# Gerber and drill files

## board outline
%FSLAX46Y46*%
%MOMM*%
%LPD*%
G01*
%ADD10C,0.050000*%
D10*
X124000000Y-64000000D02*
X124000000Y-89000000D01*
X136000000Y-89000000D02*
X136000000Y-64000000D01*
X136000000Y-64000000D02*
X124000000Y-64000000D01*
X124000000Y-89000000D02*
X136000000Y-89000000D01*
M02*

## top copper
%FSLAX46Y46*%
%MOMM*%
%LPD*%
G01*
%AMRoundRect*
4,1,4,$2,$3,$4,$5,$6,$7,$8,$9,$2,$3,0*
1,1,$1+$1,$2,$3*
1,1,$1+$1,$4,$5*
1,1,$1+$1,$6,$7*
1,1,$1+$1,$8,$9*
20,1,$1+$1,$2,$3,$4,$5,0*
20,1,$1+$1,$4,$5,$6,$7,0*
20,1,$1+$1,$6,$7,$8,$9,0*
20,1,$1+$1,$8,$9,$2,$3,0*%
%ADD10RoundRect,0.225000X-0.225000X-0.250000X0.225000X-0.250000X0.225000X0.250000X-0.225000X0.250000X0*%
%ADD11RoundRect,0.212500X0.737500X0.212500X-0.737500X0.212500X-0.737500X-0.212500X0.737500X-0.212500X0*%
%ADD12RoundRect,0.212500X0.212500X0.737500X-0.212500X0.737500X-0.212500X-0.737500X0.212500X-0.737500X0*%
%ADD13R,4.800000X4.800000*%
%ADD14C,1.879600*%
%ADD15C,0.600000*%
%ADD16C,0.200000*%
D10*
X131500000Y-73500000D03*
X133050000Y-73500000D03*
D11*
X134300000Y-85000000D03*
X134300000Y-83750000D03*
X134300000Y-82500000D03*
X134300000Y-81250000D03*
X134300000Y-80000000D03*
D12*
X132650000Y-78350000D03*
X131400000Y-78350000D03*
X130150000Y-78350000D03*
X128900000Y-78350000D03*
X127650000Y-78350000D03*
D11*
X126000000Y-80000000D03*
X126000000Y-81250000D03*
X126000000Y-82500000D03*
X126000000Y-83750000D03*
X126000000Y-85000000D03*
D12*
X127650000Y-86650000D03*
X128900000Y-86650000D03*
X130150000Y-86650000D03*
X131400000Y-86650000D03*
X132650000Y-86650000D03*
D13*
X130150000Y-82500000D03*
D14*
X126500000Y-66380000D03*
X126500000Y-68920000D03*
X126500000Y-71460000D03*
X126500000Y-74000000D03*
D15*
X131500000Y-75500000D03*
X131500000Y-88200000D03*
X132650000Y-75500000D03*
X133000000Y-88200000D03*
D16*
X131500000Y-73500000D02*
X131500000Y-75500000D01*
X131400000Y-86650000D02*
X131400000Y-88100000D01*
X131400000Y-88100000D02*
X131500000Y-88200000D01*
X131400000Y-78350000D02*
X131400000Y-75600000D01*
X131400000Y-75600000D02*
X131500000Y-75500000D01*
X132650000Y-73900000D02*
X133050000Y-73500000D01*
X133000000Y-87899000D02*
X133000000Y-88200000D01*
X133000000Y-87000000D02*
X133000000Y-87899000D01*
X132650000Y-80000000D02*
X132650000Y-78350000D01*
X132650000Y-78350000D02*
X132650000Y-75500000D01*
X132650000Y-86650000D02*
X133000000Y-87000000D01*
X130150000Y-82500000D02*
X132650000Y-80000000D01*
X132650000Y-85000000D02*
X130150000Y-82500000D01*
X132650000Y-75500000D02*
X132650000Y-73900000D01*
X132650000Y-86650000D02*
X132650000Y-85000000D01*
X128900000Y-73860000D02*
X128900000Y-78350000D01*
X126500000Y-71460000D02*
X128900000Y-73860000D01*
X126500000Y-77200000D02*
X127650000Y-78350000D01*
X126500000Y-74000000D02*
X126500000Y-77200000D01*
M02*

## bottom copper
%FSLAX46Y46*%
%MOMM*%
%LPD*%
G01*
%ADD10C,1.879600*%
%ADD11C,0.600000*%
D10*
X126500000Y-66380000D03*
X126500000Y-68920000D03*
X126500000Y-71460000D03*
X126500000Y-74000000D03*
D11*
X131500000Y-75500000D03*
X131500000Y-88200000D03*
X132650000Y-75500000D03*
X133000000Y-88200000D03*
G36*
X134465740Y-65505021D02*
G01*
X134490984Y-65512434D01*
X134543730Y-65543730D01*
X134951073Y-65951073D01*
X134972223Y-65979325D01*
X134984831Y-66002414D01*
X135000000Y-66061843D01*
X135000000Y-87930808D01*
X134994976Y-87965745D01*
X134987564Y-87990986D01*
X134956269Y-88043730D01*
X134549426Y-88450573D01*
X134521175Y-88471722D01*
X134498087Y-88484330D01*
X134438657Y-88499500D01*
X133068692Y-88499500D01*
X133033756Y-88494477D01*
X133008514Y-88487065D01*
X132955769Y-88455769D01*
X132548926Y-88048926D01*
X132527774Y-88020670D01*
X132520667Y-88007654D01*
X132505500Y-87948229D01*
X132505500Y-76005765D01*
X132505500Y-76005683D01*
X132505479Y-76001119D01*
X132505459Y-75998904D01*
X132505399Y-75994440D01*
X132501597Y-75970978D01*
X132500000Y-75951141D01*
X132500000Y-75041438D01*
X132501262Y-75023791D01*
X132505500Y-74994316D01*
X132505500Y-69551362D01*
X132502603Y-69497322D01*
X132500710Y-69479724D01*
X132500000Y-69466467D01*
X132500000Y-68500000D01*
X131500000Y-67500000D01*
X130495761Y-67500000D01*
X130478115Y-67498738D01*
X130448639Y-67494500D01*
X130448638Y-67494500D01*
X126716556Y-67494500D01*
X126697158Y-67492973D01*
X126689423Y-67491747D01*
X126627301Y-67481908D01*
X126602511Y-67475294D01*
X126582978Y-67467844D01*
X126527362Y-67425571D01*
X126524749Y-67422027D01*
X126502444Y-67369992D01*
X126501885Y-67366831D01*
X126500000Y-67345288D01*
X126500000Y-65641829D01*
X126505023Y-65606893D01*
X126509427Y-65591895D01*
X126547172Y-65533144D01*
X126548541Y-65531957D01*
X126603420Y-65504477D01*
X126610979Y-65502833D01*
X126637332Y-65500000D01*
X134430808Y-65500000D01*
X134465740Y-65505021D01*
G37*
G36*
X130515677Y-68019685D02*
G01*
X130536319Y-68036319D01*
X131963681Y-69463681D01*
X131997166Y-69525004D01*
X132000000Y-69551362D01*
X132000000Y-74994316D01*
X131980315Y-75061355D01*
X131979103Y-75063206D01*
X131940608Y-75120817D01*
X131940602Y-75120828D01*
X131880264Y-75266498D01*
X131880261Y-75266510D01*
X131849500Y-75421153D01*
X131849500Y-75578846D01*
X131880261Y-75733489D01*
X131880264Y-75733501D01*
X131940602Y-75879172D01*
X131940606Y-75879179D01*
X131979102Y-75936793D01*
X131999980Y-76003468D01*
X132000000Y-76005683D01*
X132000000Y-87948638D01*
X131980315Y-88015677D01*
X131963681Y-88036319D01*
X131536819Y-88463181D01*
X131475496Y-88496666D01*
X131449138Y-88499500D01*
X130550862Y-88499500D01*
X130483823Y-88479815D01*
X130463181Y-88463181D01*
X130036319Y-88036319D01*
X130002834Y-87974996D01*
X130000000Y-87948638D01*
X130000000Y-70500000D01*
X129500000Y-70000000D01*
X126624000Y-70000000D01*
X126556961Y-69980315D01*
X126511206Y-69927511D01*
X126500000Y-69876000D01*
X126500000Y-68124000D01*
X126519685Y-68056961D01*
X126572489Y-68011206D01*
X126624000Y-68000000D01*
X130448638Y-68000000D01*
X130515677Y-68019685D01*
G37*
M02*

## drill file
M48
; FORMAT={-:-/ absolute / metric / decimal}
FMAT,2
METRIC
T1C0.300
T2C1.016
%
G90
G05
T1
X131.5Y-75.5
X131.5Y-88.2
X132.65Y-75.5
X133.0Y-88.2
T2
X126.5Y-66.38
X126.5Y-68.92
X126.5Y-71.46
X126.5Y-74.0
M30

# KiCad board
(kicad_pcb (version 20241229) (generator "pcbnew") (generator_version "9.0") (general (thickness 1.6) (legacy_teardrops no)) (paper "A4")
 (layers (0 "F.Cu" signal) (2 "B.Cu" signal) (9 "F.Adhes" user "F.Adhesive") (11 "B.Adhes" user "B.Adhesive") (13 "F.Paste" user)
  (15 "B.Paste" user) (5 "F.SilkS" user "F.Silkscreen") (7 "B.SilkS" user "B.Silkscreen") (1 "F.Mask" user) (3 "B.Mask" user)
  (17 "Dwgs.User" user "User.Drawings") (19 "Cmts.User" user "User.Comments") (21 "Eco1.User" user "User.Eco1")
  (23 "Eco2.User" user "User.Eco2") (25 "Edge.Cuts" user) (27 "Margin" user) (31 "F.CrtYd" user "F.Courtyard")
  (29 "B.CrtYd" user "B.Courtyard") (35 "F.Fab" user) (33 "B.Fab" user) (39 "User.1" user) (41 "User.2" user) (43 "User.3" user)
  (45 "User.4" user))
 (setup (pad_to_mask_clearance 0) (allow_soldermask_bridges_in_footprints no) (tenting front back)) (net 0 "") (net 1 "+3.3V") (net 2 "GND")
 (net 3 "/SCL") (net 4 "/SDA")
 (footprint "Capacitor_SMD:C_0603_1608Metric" (layer "F.Cu") (at 132.275 73.5)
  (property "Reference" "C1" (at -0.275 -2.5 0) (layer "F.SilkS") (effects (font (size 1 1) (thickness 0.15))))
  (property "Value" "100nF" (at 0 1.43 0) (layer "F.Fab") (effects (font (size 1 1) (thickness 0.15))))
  (pad "1" smd roundrect (at -0.775 0) (size 0.9 0.95) (layers "F.Cu" "F.Mask" "F.Paste") (roundrect_rratio 0.25) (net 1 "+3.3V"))
  (pad "2" smd roundrect (at 0.775 0) (size 0.9 0.95) (layers "F.Cu" "F.Mask" "F.Paste") (roundrect_rratio 0.25) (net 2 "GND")))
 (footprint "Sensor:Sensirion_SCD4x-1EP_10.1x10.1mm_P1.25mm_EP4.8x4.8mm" (layer "F.Cu") (at 130.15 82.5 180)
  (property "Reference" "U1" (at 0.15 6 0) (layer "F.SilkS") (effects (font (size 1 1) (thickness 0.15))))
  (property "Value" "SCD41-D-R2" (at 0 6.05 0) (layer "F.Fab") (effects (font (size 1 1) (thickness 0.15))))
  (pad "" smd roundrect (at -1.2 -1.2 180) (size 1.93 1.93) (layers "F.Paste") (roundrect_rratio 0.129534))
  (pad "" smd roundrect (at -1.2 1.2 180) (size 1.93 1.93) (layers "F.Paste") (roundrect_rratio 0.129534))
  (pad "" smd roundrect (at 1.2 -1.2 180) (size 1.93 1.93) (layers "F.Paste") (roundrect_rratio 0.129534))
  (pad "" smd roundrect (at 1.2 1.2 180) (size 1.93 1.93) (layers "F.Paste") (roundrect_rratio 0.129534))
  (pad "1" smd roundrect (at -4.15 -2.5 180) (size 1.9 0.85) (layers "F.Cu" "F.Mask" "F.Paste") (roundrect_rratio 0.25))
  (pad "2" smd roundrect (at -4.15 -1.25 180) (size 1.9 0.85) (layers "F.Cu" "F.Mask" "F.Paste") (roundrect_rratio 0.25))
  (pad "3" smd roundrect (at -4.15 0 180) (size 1.9 0.85) (layers "F.Cu" "F.Mask" "F.Paste") (roundrect_rratio 0.25))
  (pad "4" smd roundrect (at -4.15 1.25 180) (size 1.9 0.85) (layers "F.Cu" "F.Mask" "F.Paste") (roundrect_rratio 0.25))
  (pad "5" smd roundrect (at -4.15 2.5 180) (size 1.9 0.85) (layers "F.Cu" "F.Mask" "F.Paste") (roundrect_rratio 0.25))
  (pad "6" smd roundrect (at -2.5 4.15 180) (size 0.85 1.9) (layers "F.Cu" "F.Mask" "F.Paste") (roundrect_rratio 0.25) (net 2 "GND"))
  (pad "7" smd roundrect (at -1.25 4.15 180) (size 0.85 1.9) (layers "F.Cu" "F.Mask" "F.Paste") (roundrect_rratio 0.25) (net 1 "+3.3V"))
  (pad "8" smd roundrect (at 0 4.15 180) (size 0.85 1.9) (layers "F.Cu" "F.Mask" "F.Paste") (roundrect_rratio 0.25))
  (pad "9" smd roundrect (at 1.25 4.15 180) (size 0.85 1.9) (layers "F.Cu" "F.Mask" "F.Paste") (roundrect_rratio 0.25) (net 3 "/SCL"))
  (pad "10" smd roundrect (at 2.5 4.15 180) (size 0.85 1.9) (layers "F.Cu" "F.Mask" "F.Paste") (roundrect_rratio 0.25) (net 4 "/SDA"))
  (pad "11" smd roundrect (at 4.15 2.5 180) (size 1.9 0.85) (layers "F.Cu" "F.Mask" "F.Paste") (roundrect_rratio 0.25))
  (pad "12" smd roundrect (at 4.15 1.25 180) (size 1.9 0.85) (layers "F.Cu" "F.Mask" "F.Paste") (roundrect_rratio 0.25))
  (pad "13" smd roundrect (at 4.15 0 180) (size 1.9 0.85) (layers "F.Cu" "F.Mask" "F.Paste") (roundrect_rratio 0.25))
  (pad "14" smd roundrect (at 4.15 -1.25 180) (size 1.9 0.85) (layers "F.Cu" "F.Mask" "F.Paste") (roundrect_rratio 0.25))
  (pad "15" smd roundrect (at 4.15 -2.5 180) (size 1.9 0.85) (layers "F.Cu" "F.Mask" "F.Paste") (roundrect_rratio 0.25))
  (pad "16" smd roundrect (at 2.5 -4.15 180) (size 0.85 1.9) (layers "F.Cu" "F.Mask" "F.Paste") (roundrect_rratio 0.25))
  (pad "17" smd roundrect (at 1.25 -4.15 180) (size 0.85 1.9) (layers "F.Cu" "F.Mask" "F.Paste") (roundrect_rratio 0.25))
  (pad "18" smd roundrect (at 0 -4.15 180) (size 0.85 1.9) (layers "F.Cu" "F.Mask" "F.Paste") (roundrect_rratio 0.25))
  (pad "19" smd roundrect (at -1.25 -4.15 180) (size 0.85 1.9) (layers "F.Cu" "F.Mask" "F.Paste") (roundrect_rratio 0.25) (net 1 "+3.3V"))
  (pad "20" smd roundrect (at -2.5 -4.15 180) (size 0.85 1.9) (layers "F.Cu" "F.Mask" "F.Paste") (roundrect_rratio 0.25) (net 2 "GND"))
  (pad "21" smd rect (at 0 0 180) (size 4.8 4.8) (layers "F.Cu" "F.Mask") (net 2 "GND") (zone_connect 2)))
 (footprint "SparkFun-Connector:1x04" (layer "F.Cu") (at 126.5 66.38 -90)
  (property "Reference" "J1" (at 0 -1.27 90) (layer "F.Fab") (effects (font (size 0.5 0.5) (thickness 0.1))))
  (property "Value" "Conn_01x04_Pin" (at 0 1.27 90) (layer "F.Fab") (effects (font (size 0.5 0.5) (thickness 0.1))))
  (pad "1" thru_hole circle (at 0 0) (size 1.8796 1.8796) (drill 1.016) (layers "*.Cu" "*.Mask") (remove_unused_layers yes)
   (keep_end_layers yes) (zone_layer_connections) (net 2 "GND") (thermal_bridge_angle 0))
  (pad "2" thru_hole circle (at 2.54 0) (size 1.8796 1.8796) (drill 1.016) (layers "*.Cu" "*.Mask") (remove_unused_layers yes)
   (keep_end_layers yes) (zone_layer_connections) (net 1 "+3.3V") (thermal_bridge_angle 0))
  (pad "3" thru_hole circle (at 5.08 0) (size 1.8796 1.8796) (drill 1.016) (layers "*.Cu" "*.Mask") (remove_unused_layers yes)
   (keep_end_layers yes) (zone_layer_connections) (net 3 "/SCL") (thermal_bridge_angle 0))
  (pad "4" thru_hole circle (at 7.62 0) (size 1.8796 1.8796) (drill 1.016) (layers "*.Cu" "*.Mask") (remove_unused_layers yes)
   (keep_end_layers yes) (zone_layer_connections) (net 4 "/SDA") (thermal_bridge_angle 0)))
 (gr_line (start 124 64) (end 124 89) (stroke (width 0.05) (type default)) (layer "Edge.Cuts"))
 (gr_line (start 136 89) (end 136 64) (stroke (width 0.05) (type default)) (layer "Edge.Cuts"))
 (gr_line (start 136 64) (end 124 64) (stroke (width 0.05) (type default)) (layer "Edge.Cuts"))
 (gr_line (start 124 89) (end 136 89) (stroke (width 0.05) (type default)) (layer "Edge.Cuts"))
 (segment (start 131.5 73.5) (end 131.5 75.5) (width 0.2) (layer "F.Cu") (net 1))
 (segment (start 131.4 86.65) (end 131.4 88.1) (width 0.2) (layer "F.Cu") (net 1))
 (segment (start 131.4 88.1) (end 131.5 88.2) (width 0.2) (layer "F.Cu") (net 1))
 (segment (start 131.4 78.35) (end 131.4 75.6) (width 0.2) (layer "F.Cu") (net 1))
 (segment (start 131.4 75.6) (end 131.5 75.5) (width 0.2) (layer "F.Cu") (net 1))
 (via (at 131.5 75.5) (size 0.6) (drill 0.3) (layers "F.Cu" "B.Cu") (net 1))
 (via (at 131.5 88.2) (size 0.6) (drill 0.3) (layers "F.Cu" "B.Cu") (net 1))
 (segment (start 132.65 73.9) (end 133.05 73.5) (width 0.2) (layer "F.Cu") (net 2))
 (segment (start 133 87.899) (end 133 88.2) (width 0.2) (layer "F.Cu") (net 2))
 (segment (start 133 87) (end 133 87.899) (width 0.2) (layer "F.Cu") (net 2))
 (segment (start 132.65 80) (end 132.65 78.35) (width 0.2) (layer "F.Cu") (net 2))
 (segment (start 132.65 78.35) (end 132.65 75.5) (width 0.2) (layer "F.Cu") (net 2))
 (segment (start 132.65 86.65) (end 133 87) (width 0.2) (layer "F.Cu") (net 2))
 (segment (start 130.15 82.5) (end 132.65 80) (width 0.2) (layer "F.Cu") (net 2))
 (segment (start 132.65 85) (end 130.15 82.5) (width 0.2) (layer "F.Cu") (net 2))
 (segment (start 132.65 75.5) (end 132.65 73.9) (width 0.2) (layer "F.Cu") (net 2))
 (segment (start 132.65 86.65) (end 132.65 85) (width 0.2) (layer "F.Cu") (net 2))
 (via (at 132.65 75.5) (size 0.6) (drill 0.3) (layers "F.Cu" "B.Cu") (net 2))
 (via (at 133 88.2) (size 0.6) (drill 0.3) (layers "F.Cu" "B.Cu") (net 2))
 (segment (start 128.9 73.86) (end 128.9 78.35) (width 0.2) (layer "F.Cu") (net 3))
 (segment (start 126.5 71.46) (end 128.9 73.86) (width 0.2) (layer "F.Cu") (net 3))
 (segment (start 126.5 77.2) (end 127.65 78.35) (width 0.2) (layer "F.Cu") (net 4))
 (segment (start 126.5 74) (end 126.5 77.2) (width 0.2) (layer "F.Cu") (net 4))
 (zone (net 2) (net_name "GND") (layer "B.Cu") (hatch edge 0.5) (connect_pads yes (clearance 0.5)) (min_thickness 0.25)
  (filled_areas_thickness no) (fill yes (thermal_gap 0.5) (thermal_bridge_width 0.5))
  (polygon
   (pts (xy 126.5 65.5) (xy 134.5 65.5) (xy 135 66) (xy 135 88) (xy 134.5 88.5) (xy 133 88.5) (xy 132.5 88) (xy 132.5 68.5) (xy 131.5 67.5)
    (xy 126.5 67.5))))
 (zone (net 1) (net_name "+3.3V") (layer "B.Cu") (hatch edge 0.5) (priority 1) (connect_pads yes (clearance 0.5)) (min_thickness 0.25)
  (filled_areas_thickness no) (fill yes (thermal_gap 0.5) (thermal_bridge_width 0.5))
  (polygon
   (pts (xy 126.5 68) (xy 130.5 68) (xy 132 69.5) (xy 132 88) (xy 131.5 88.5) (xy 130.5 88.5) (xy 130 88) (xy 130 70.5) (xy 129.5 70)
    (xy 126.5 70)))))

